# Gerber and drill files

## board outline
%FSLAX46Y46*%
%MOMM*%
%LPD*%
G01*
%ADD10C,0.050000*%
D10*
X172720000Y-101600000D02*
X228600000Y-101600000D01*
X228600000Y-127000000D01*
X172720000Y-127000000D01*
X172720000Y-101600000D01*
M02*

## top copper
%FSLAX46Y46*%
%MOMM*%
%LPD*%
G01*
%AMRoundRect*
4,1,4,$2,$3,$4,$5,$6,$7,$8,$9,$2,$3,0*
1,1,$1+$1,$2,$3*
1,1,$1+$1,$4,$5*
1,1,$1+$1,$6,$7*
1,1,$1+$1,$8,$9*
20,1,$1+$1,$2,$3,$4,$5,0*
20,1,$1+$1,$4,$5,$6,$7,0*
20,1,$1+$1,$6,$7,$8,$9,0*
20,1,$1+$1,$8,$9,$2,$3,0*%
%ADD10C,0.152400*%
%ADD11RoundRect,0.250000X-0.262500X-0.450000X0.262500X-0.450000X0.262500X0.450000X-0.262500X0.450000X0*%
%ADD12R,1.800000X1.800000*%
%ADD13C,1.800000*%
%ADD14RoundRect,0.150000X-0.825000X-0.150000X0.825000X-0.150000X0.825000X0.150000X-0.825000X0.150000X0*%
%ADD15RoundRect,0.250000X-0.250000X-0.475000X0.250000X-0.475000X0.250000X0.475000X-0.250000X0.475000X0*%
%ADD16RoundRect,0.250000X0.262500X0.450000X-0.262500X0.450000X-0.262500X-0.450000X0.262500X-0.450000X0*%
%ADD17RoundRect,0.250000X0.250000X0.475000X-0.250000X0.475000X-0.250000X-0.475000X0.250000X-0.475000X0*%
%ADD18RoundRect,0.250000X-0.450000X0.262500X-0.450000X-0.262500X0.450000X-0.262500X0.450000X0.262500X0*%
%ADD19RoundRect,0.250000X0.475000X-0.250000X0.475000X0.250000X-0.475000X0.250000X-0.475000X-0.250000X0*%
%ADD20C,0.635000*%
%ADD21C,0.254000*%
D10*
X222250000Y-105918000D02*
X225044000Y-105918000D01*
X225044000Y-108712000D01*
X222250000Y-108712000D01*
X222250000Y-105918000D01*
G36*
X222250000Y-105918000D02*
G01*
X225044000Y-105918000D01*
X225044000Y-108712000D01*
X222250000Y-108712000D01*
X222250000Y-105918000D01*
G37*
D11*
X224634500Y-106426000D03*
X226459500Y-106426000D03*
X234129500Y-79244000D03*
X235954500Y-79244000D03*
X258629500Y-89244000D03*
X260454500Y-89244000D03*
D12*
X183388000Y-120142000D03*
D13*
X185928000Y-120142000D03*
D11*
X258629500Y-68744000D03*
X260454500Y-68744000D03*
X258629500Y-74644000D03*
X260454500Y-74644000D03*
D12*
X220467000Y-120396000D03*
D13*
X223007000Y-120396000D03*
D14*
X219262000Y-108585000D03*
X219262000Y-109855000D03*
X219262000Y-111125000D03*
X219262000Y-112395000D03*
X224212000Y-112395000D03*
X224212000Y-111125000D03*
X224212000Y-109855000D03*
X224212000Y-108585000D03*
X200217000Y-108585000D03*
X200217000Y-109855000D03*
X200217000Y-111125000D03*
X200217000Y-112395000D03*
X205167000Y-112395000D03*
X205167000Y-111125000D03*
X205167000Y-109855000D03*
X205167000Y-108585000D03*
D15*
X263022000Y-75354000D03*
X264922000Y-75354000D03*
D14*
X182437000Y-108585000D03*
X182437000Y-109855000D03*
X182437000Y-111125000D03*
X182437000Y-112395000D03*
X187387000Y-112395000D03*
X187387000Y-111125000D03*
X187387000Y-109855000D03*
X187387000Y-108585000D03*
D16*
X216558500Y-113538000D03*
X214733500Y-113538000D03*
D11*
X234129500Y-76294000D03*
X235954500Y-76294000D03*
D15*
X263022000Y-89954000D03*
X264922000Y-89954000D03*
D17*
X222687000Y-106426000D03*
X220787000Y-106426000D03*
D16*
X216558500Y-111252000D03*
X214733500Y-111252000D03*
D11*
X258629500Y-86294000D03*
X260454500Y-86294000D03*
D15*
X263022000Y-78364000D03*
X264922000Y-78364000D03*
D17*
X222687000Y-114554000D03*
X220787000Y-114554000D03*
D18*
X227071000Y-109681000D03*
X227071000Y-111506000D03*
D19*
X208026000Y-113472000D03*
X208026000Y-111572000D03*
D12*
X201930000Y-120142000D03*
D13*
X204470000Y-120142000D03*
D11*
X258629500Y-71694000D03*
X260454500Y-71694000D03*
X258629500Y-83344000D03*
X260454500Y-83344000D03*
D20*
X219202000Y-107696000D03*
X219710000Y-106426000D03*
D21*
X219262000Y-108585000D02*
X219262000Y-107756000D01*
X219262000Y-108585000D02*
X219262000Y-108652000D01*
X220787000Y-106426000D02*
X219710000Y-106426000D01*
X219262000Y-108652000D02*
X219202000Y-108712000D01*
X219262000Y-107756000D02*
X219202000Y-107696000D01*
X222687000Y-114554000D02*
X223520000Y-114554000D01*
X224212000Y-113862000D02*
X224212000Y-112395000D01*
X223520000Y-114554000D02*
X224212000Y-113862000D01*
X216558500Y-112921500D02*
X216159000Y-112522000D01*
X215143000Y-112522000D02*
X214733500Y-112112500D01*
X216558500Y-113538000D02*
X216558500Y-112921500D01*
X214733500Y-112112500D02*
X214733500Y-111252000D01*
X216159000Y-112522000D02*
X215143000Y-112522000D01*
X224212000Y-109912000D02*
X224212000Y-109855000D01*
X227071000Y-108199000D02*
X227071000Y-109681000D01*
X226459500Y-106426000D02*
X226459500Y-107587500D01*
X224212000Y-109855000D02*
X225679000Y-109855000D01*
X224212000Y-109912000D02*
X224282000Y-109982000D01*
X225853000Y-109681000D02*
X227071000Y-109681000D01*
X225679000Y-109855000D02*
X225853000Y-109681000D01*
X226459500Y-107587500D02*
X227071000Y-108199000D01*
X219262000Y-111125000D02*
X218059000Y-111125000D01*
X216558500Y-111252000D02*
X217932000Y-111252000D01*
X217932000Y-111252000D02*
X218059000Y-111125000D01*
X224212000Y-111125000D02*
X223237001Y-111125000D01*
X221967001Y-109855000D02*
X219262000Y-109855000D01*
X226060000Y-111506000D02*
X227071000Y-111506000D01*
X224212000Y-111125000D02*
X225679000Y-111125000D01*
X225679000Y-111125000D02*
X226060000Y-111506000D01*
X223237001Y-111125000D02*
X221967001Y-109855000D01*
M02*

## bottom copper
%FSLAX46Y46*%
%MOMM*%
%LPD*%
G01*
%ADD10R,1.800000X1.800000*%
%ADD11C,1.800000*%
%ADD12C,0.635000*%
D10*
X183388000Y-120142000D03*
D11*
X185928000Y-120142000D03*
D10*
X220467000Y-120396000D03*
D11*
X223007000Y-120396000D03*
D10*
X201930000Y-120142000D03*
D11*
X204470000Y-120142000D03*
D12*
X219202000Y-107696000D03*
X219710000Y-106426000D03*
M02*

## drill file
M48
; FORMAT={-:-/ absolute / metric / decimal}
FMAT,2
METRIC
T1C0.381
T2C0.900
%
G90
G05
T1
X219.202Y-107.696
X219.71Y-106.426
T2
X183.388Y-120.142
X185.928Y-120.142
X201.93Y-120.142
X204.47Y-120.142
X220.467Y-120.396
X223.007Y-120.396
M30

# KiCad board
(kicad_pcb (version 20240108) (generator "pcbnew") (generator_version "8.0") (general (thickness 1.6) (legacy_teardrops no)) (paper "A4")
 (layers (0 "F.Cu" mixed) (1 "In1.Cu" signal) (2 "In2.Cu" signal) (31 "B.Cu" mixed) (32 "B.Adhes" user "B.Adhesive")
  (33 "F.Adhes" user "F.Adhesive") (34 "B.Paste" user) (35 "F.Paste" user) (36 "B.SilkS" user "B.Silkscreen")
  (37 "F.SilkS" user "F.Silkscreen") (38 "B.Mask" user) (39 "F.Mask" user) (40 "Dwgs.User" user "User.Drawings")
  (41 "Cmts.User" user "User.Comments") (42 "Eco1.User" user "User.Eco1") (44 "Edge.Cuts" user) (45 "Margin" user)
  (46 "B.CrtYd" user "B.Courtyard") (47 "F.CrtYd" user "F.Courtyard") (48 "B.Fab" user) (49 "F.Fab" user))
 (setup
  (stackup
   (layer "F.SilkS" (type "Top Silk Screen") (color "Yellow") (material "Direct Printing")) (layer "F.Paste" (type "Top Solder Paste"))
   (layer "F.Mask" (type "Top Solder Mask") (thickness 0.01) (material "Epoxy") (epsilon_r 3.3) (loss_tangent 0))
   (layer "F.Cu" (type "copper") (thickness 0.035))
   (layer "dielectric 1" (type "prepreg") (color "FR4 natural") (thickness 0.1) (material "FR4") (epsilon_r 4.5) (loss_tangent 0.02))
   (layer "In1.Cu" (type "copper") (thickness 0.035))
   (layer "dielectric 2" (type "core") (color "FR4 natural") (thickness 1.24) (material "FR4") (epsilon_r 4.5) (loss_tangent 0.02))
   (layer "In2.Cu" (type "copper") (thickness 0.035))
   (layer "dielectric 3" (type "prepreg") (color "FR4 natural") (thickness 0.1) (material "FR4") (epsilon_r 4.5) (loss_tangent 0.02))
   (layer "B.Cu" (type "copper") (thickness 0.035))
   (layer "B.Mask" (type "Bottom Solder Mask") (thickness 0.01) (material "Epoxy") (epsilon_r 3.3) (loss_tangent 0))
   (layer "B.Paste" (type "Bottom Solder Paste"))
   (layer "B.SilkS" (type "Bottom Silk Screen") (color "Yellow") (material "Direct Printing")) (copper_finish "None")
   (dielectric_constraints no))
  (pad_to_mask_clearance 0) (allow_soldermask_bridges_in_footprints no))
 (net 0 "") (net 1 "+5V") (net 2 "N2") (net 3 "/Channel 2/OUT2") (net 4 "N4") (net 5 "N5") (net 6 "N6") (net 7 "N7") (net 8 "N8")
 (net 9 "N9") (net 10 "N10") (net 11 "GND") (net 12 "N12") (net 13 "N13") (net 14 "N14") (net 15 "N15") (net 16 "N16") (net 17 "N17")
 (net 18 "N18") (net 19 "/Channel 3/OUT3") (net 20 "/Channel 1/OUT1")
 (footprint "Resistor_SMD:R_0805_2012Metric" (layer "F.Cu") (at 225.547 106.426)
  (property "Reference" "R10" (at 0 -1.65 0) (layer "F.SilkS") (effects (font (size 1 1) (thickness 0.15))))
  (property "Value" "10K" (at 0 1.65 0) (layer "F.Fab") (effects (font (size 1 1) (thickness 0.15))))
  (pad "1" smd roundrect (at -0.9125 0) (size 1.025 1.4) (layers "F.Cu" "F.Paste" "F.Mask") (roundrect_rratio 0.243902) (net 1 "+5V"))
  (pad "2" smd roundrect (at 0.9125 0) (size 1.025 1.4) (layers "F.Cu" "F.Paste" "F.Mask") (roundrect_rratio 0.243902) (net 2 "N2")))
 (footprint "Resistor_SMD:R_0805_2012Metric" (layer "F.Cu") (at 235.042 79.244)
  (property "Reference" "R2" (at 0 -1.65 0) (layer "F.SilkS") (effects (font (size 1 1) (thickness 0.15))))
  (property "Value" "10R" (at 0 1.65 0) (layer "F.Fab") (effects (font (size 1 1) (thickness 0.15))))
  (pad "1" smd roundrect (at -0.9125 0) (size 1.025 1.4) (layers "F.Cu" "F.Paste" "F.Mask") (roundrect_rratio 0.243902)
   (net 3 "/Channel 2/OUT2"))
  (pad "2" smd roundrect (at 0.9125 0) (size 1.025 1.4) (layers "F.Cu" "F.Paste" "F.Mask") (roundrect_rratio 0.243902) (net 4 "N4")))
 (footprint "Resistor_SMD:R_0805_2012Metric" (layer "F.Cu") (at 259.542 89.244)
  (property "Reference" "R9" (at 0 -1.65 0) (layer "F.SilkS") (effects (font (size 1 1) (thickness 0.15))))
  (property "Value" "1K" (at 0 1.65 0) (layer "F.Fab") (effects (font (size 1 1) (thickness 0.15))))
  (pad "1" smd roundrect (at -0.9125 0) (size 1.025 1.4) (layers "F.Cu" "F.Paste" "F.Mask") (roundrect_rratio 0.243902) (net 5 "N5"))
  (pad "2" smd roundrect (at 0.9125 0) (size 1.025 1.4) (layers "F.Cu" "F.Paste" "F.Mask") (roundrect_rratio 0.243902) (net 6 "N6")))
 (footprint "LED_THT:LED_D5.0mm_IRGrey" (layer "F.Cu") (at 183.388 120.142)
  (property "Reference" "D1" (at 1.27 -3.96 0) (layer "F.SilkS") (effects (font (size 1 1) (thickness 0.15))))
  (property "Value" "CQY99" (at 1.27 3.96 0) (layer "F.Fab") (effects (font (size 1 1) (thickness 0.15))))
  (pad "1" thru_hole rect (at 0 0) (size 1.8 1.8) (drill 0.9) (layers "*.Cu" "*.Mask") (remove_unused_layers no) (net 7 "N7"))
  (pad "2" thru_hole circle (at 2.54 0) (size 1.8 1.8) (drill 0.9) (layers "*.Cu" "*.Mask") (remove_unused_layers no) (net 1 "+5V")))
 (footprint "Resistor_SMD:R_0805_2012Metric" (layer "F.Cu") (at 259.542 68.744)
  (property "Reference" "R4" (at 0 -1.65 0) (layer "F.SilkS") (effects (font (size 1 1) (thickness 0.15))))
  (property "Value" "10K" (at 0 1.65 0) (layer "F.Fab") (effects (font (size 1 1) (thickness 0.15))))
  (pad "1" smd roundrect (at -0.9125 0) (size 1.025 1.4) (layers "F.Cu" "F.Paste" "F.Mask") (roundrect_rratio 0.243902) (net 1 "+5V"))
  (pad "2" smd roundrect (at 0.9125 0) (size 1.025 1.4) (layers "F.Cu" "F.Paste" "F.Mask") (roundrect_rratio 0.243902) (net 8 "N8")))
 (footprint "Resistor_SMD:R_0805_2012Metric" (layer "F.Cu") (at 259.542 74.644)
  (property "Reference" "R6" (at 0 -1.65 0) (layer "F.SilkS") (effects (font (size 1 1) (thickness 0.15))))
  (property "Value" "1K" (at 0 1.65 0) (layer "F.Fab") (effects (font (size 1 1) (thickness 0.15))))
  (pad "1" smd roundrect (at -0.9125 0) (size 1.025 1.4) (layers "F.Cu" "F.Paste" "F.Mask") (roundrect_rratio 0.243902) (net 8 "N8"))
  (pad "2" smd roundrect (at 0.9125 0) (size 1.025 1.4) (layers "F.Cu" "F.Paste" "F.Mask") (roundrect_rratio 0.243902) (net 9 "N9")))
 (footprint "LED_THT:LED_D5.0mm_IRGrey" (layer "F.Cu") (at 220.467 120.396)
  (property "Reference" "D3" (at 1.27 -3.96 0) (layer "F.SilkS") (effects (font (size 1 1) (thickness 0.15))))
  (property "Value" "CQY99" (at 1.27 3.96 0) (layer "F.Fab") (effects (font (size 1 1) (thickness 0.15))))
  (pad "1" thru_hole rect (at 0 0) (size 1.8 1.8) (drill 0.9) (layers "*.Cu" "*.Mask") (remove_unused_layers no) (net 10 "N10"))
  (pad "2" thru_hole circle (at 2.54 0) (size 1.8 1.8) (drill 0.9) (layers "*.Cu" "*.Mask") (remove_unused_layers no) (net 1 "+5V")))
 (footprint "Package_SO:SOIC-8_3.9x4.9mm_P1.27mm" (layer "F.Cu") (at 221.737 110.49)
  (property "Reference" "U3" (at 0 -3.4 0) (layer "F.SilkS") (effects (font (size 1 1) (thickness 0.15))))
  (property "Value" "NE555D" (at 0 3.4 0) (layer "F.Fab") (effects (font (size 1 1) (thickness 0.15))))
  (pad "1" smd roundrect (at -2.475 -1.905) (size 1.95 0.6) (layers "F.Cu" "F.Paste" "F.Mask") (roundrect_rratio 0.25) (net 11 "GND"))
  (pad "2" smd roundrect (at -2.475 -0.635) (size 1.95 0.6) (layers "F.Cu" "F.Paste" "F.Mask") (roundrect_rratio 0.25) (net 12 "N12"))
  (pad "3" smd roundrect (at -2.475 0.635) (size 1.95 0.6) (layers "F.Cu" "F.Paste" "F.Mask") (roundrect_rratio 0.25) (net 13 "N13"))
  (pad "4" smd roundrect (at -2.475 1.905) (size 1.95 0.6) (layers "F.Cu" "F.Paste" "F.Mask") (roundrect_rratio 0.25) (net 1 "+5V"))
  (pad "5" smd roundrect (at 2.475 1.905) (size 1.95 0.6) (layers "F.Cu" "F.Paste" "F.Mask") (roundrect_rratio 0.25) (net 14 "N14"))
  (pad "6" smd roundrect (at 2.475 0.635) (size 1.95 0.6) (layers "F.Cu" "F.Paste" "F.Mask") (roundrect_rratio 0.25) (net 12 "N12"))
  (pad "7" smd roundrect (at 2.475 -0.635) (size 1.95 0.6) (layers "F.Cu" "F.Paste" "F.Mask") (roundrect_rratio 0.25) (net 2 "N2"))
  (pad "8" smd roundrect (at 2.475 -1.905) (size 1.95 0.6) (layers "F.Cu" "F.Paste" "F.Mask") (roundrect_rratio 0.25) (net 1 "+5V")))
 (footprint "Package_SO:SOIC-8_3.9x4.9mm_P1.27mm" (layer "F.Cu") (at 202.692 110.49)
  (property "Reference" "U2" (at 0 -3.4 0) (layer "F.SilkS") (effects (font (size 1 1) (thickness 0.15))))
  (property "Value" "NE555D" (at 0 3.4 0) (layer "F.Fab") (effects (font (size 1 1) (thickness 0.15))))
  (pad "1" smd roundrect (at -2.475 -1.905) (size 1.95 0.6) (layers "F.Cu" "F.Paste" "F.Mask") (roundrect_rratio 0.25) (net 11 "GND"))
  (pad "2" smd roundrect (at -2.475 -0.635) (size 1.95 0.6) (layers "F.Cu" "F.Paste" "F.Mask") (roundrect_rratio 0.25) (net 6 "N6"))
  (pad "3" smd roundrect (at -2.475 0.635) (size 1.95 0.6) (layers "F.Cu" "F.Paste" "F.Mask") (roundrect_rratio 0.25) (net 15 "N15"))
  (pad "4" smd roundrect (at -2.475 1.905) (size 1.95 0.6) (layers "F.Cu" "F.Paste" "F.Mask") (roundrect_rratio 0.25) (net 1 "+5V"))
  (pad "5" smd roundrect (at 2.475 1.905) (size 1.95 0.6) (layers "F.Cu" "F.Paste" "F.Mask") (roundrect_rratio 0.25) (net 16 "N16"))
  (pad "6" smd roundrect (at 2.475 0.635) (size 1.95 0.6) (layers "F.Cu" "F.Paste" "F.Mask") (roundrect_rratio 0.25) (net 6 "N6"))
  (pad "7" smd roundrect (at 2.475 -0.635) (size 1.95 0.6) (layers "F.Cu" "F.Paste" "F.Mask") (roundrect_rratio 0.25) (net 5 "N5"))
  (pad "8" smd roundrect (at 2.475 -1.905) (size 1.95 0.6) (layers "F.Cu" "F.Paste" "F.Mask") (roundrect_rratio 0.25) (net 1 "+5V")))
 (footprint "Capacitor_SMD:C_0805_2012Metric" (layer "F.Cu") (at 263.972 75.354)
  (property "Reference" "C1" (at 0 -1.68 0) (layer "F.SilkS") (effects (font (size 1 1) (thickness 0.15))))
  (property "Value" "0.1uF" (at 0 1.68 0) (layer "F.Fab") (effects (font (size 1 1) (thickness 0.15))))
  (pad "1" smd roundrect (at -0.95 0) (size 1 1.45) (layers "F.Cu" "F.Paste" "F.Mask") (roundrect_rratio 0.25) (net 1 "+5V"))
  (pad "2" smd roundrect (at 0.95 0) (size 1 1.45) (layers "F.Cu" "F.Paste" "F.Mask") (roundrect_rratio 0.25) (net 11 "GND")))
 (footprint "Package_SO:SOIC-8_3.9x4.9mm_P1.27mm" (layer "F.Cu") (at 184.912 110.49)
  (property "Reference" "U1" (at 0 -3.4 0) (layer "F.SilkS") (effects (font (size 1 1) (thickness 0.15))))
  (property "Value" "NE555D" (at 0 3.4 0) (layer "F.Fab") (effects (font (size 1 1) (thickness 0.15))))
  (pad "1" smd roundrect (at -2.475 -1.905) (size 1.95 0.6) (layers "F.Cu" "F.Paste" "F.Mask") (roundrect_rratio 0.25) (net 11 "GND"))
  (pad "2" smd roundrect (at -2.475 -0.635) (size 1.95 0.6) (layers "F.Cu" "F.Paste" "F.Mask") (roundrect_rratio 0.25) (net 9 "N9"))
  (pad "3" smd roundrect (at -2.475 0.635) (size 1.95 0.6) (layers "F.Cu" "F.Paste" "F.Mask") (roundrect_rratio 0.25) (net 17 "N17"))
  (pad "4" smd roundrect (at -2.475 1.905) (size 1.95 0.6) (layers "F.Cu" "F.Paste" "F.Mask") (roundrect_rratio 0.25) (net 1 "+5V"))
  (pad "5" smd roundrect (at 2.475 1.905) (size 1.95 0.6) (layers "F.Cu" "F.Paste" "F.Mask") (roundrect_rratio 0.25) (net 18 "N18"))
  (pad "6" smd roundrect (at 2.475 0.635) (size 1.95 0.6) (layers "F.Cu" "F.Paste" "F.Mask") (roundrect_rratio 0.25) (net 9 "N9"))
  (pad "7" smd roundrect (at 2.475 -0.635) (size 1.95 0.6) (layers "F.Cu" "F.Paste" "F.Mask") (roundrect_rratio 0.25) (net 8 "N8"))
  (pad "8" smd roundrect (at 2.475 -1.905) (size 1.95 0.6) (layers "F.Cu" "F.Paste" "F.Mask") (roundrect_rratio 0.25) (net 1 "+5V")))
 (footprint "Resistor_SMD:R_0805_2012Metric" (layer "F.Cu") (at 215.646 113.538 180)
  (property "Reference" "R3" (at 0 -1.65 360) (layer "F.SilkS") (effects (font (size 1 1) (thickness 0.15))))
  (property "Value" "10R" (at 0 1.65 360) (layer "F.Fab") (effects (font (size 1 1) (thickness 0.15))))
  (pad "1" smd roundrect (at -0.9125 0 180) (size 1.025 1.4) (layers "F.Cu" "F.Paste" "F.Mask") (roundrect_rratio 0.243902)
   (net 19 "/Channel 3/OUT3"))
  (pad "2" smd roundrect (at 0.9125 0 180) (size 1.025 1.4) (layers "F.Cu" "F.Paste" "F.Mask") (roundrect_rratio 0.243902) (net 10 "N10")))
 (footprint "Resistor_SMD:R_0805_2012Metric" (layer "F.Cu") (at 235.042 76.294)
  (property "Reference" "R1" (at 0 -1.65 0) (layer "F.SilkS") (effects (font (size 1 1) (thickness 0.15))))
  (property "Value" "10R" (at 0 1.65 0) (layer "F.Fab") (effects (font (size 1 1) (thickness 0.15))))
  (pad "1" smd roundrect (at -0.9125 0) (size 1.025 1.4) (layers "F.Cu" "F.Paste" "F.Mask") (roundrect_rratio 0.243902)
   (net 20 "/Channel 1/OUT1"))
  (pad "2" smd roundrect (at 0.9125 0) (size 1.025 1.4) (layers "F.Cu" "F.Paste" "F.Mask") (roundrect_rratio 0.243902) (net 7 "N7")))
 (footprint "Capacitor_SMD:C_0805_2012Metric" (layer "F.Cu") (at 263.972 89.954)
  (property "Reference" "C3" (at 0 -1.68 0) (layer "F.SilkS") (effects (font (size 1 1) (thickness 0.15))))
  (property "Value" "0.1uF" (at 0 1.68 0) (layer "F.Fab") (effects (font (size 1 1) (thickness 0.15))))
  (pad "1" smd roundrect (at -0.95 0) (size 1 1.45) (layers "F.Cu" "F.Paste" "F.Mask") (roundrect_rratio 0.25) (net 1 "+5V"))
  (pad "2" smd roundrect (at 0.95 0) (size 1 1.45) (layers "F.Cu" "F.Paste" "F.Mask") (roundrect_rratio 0.25) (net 11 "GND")))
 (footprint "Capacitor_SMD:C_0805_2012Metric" (layer "F.Cu") (at 221.737 106.426 180)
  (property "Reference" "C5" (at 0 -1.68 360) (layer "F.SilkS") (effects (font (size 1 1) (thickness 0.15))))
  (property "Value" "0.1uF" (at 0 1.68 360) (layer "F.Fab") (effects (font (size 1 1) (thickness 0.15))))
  (pad "1" smd roundrect (at -0.95 0 180) (size 1 1.45) (layers "F.Cu" "F.Paste" "F.Mask") (roundrect_rratio 0.25) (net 1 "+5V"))
  (pad "2" smd roundrect (at 0.95 0 180) (size 1 1.45) (layers "F.Cu" "F.Paste" "F.Mask") (roundrect_rratio 0.25) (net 11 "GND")))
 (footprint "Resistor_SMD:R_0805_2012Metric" (layer "F.Cu") (at 215.646 111.252 180)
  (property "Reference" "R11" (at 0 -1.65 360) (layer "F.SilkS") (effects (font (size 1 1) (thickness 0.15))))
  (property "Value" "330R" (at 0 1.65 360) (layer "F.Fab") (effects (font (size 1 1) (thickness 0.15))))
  (pad "1" smd roundrect (at -0.9125 0 180) (size 1.025 1.4) (layers "F.Cu" "F.Paste" "F.Mask") (roundrect_rratio 0.243902) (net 13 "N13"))
  (pad "2" smd roundrect (at 0.9125 0 180) (size 1.025 1.4) (layers "F.Cu" "F.Paste" "F.Mask") (roundrect_rratio 0.243902)
   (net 19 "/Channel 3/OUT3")))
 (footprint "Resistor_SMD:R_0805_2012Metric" (layer "F.Cu") (at 259.542 86.294)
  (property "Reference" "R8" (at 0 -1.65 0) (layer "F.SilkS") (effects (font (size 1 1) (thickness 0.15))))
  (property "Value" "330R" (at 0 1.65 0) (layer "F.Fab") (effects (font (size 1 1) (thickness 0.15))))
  (pad "1" smd roundrect (at -0.9125 0) (size 1.025 1.4) (layers "F.Cu" "F.Paste" "F.Mask") (roundrect_rratio 0.243902) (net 15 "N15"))
  (pad "2" smd roundrect (at 0.9125 0) (size 1.025 1.4) (layers "F.Cu" "F.Paste" "F.Mask") (roundrect_rratio 0.243902)
   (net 3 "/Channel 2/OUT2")))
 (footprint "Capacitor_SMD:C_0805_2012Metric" (layer "F.Cu") (at 263.972 78.364)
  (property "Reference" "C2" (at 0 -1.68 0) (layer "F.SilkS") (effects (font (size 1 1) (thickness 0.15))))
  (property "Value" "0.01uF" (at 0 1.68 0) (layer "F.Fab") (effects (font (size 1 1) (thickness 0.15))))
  (pad "1" smd roundrect (at -0.95 0) (size 1 1.45) (layers "F.Cu" "F.Paste" "F.Mask") (roundrect_rratio 0.25) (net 18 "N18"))
  (pad "2" smd roundrect (at 0.95 0) (size 1 1.45) (layers "F.Cu" "F.Paste" "F.Mask") (roundrect_rratio 0.25) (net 11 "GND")))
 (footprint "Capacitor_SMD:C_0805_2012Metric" (layer "F.Cu") (at 221.737 114.554 180)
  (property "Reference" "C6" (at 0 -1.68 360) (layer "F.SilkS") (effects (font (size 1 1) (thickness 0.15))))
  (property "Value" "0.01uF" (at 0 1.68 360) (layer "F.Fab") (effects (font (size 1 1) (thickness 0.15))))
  (pad "1" smd roundrect (at -0.95 0 180) (size 1 1.45) (layers "F.Cu" "F.Paste" "F.Mask") (roundrect_rratio 0.25) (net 14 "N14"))
  (pad "2" smd roundrect (at 0.95 0 180) (size 1 1.45) (layers "F.Cu" "F.Paste" "F.Mask") (roundrect_rratio 0.25) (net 11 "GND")))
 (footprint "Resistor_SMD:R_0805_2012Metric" (layer "F.Cu") (at 227.071 110.5935 -90)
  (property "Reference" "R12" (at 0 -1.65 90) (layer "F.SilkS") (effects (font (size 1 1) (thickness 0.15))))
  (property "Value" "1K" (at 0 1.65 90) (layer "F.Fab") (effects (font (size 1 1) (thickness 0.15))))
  (pad "1" smd roundrect (at -0.9125 0 270) (size 1.025 1.4) (layers "F.Cu" "F.Paste" "F.Mask") (roundrect_rratio 0.243902) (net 2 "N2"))
  (pad "2" smd roundrect (at 0.9125 0 270) (size 1.025 1.4) (layers "F.Cu" "F.Paste" "F.Mask") (roundrect_rratio 0.243902) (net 12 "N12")))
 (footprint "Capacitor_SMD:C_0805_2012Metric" (layer "F.Cu") (at 208.026 112.522 90)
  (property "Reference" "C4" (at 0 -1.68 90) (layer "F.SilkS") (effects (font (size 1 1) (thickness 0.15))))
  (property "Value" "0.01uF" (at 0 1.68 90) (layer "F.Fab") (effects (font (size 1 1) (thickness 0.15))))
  (pad "1" smd roundrect (at -0.95 0 90) (size 1 1.45) (layers "F.Cu" "F.Paste" "F.Mask") (roundrect_rratio 0.25) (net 16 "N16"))
  (pad "2" smd roundrect (at 0.95 0 90) (size 1 1.45) (layers "F.Cu" "F.Paste" "F.Mask") (roundrect_rratio 0.25) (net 11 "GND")))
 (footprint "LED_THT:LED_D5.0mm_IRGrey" (layer "F.Cu") (at 201.93 120.142)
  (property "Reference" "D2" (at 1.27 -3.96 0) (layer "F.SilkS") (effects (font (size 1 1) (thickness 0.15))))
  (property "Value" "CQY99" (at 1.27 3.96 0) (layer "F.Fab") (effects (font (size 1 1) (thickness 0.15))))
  (pad "1" thru_hole rect (at 0 0) (size 1.8 1.8) (drill 0.9) (layers "*.Cu" "*.Mask") (remove_unused_layers no) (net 4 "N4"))
  (pad "2" thru_hole circle (at 2.54 0) (size 1.8 1.8) (drill 0.9) (layers "*.Cu" "*.Mask") (remove_unused_layers no) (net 1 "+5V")))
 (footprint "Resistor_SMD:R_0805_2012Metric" (layer "F.Cu") (at 259.542 71.694)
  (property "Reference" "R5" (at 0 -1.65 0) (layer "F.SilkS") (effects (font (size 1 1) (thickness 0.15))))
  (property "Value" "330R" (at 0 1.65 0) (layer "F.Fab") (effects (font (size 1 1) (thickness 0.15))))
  (pad "1" smd roundrect (at -0.9125 0) (size 1.025 1.4) (layers "F.Cu" "F.Paste" "F.Mask") (roundrect_rratio 0.243902) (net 17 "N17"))
  (pad "2" smd roundrect (at 0.9125 0) (size 1.025 1.4) (layers "F.Cu" "F.Paste" "F.Mask") (roundrect_rratio 0.243902)
   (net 20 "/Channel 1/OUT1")))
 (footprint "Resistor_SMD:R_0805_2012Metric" (layer "F.Cu") (at 259.542 83.344)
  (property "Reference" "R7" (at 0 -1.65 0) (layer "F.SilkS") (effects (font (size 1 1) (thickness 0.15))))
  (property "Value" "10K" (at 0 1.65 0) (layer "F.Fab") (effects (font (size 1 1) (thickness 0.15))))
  (pad "1" smd roundrect (at -0.9125 0) (size 1.025 1.4) (layers "F.Cu" "F.Paste" "F.Mask") (roundrect_rratio 0.243902) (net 1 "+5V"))
  (pad "2" smd roundrect (at 0.9125 0) (size 1.025 1.4) (layers "F.Cu" "F.Paste" "F.Mask") (roundrect_rratio 0.243902) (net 5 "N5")))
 (gr_rect (start 222.25 105.918) (end 225.044 108.712) (stroke (width 0.1524) (type solid)) (fill solid) (layer "F.Cu") (net 1))
 (gr_rect (start 172.72 101.6) (end 228.6 127) (stroke (width 0.05) (type default)) (fill none) (layer "Edge.Cuts"))
 (segment (start 219.262 108.585) (end 219.262 107.756) (width 0.254) (layer "F.Cu") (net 11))
 (segment (start 219.262 108.585) (end 219.262 108.652) (width 0.254) (layer "F.Cu") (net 11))
 (segment (start 220.787 106.426) (end 219.71 106.426) (width 0.254) (layer "F.Cu") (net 11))
 (segment (start 219.262 108.652) (end 219.202 108.712) (width 0.254) (layer "F.Cu") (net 11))
 (segment (start 219.262 107.756) (end 219.202 107.696) (width 0.254) (layer "F.Cu") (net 11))
 (via (at 219.202 107.696) (size 0.635) (drill 0.381) (layers "F.Cu" "B.Cu") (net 11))
 (via (at 219.71 106.426) (size 0.635) (drill 0.381) (layers "F.Cu" "B.Cu")
  (teardrops (best_length_ratio 0.5) (max_length 1) (best_width_ratio 1) (max_width 2) (curve_points 0) (filter_ratio 0.9) (enabled no)
   (allow_two_segments no) (prefer_zone_connections yes))
  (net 11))
 (segment (start 222.687 114.554) (end 223.52 114.554) (width 0.254) (layer "F.Cu") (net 14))
 (segment (start 224.212 113.862) (end 224.212 112.395) (width 0.254) (layer "F.Cu") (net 14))
 (segment (start 223.52 114.554) (end 224.212 113.862) (width 0.254) (layer "F.Cu") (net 14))
 (segment (start 216.5585 112.9215) (end 216.159 112.522) (width 0.254) (layer "F.Cu") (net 19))
 (segment (start 215.143 112.522) (end 214.7335 112.1125) (width 0.254) (layer "F.Cu") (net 19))
 (segment (start 216.5585 113.538) (end 216.5585 112.9215) (width 0.254) (layer "F.Cu") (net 19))
 (segment (start 214.7335 112.1125) (end 214.7335 111.252) (width 0.254) (layer "F.Cu") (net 19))
 (segment (start 216.159 112.522) (end 215.143 112.522) (width 0.254) (layer "F.Cu") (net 19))
 (segment (start 224.212 109.912) (end 224.212 109.855) (width 0.254) (layer "F.Cu") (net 2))
 (segment (start 227.071 108.199) (end 227.071 109.681) (width 0.254) (layer "F.Cu") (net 2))
 (segment (start 226.4595 106.426) (end 226.4595 107.5875) (width 0.254) (layer "F.Cu") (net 2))
 (segment (start 224.212 109.855) (end 225.679 109.855) (width 0.254) (layer "F.Cu") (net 2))
 (segment (start 224.212 109.912) (end 224.282 109.982) (width 0.254) (layer "F.Cu") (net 2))
 (segment (start 225.853 109.681) (end 227.071 109.681) (width 0.254) (layer "F.Cu") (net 2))
 (segment (start 225.679 109.855) (end 225.853 109.681) (width 0.254) (layer "F.Cu") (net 2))
 (segment (start 226.4595 107.5875) (end 227.071 108.199) (width 0.254) (layer "F.Cu") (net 2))
 (segment (start 219.262 111.125) (end 218.059 111.125) (width 0.254) (layer "F.Cu") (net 13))
 (segment (start 216.5585 111.252) (end 217.932 111.252) (width 0.254) (layer "F.Cu") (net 13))
 (segment (start 217.932 111.252) (end 218.059 111.125) (width 0.254) (layer "F.Cu") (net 13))
 (segment (start 224.212 111.125) (end 223.237001 111.125) (width 0.254) (layer "F.Cu") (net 12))
 (segment (start 221.967001 109.855) (end 219.262 109.855) (width 0.254) (layer "F.Cu") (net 12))
 (segment (start 226.06 111.506) (end 227.071 111.506) (width 0.254) (layer "F.Cu") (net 12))
 (segment (start 224.212 111.125) (end 225.679 111.125) (width 0.254) (layer "F.Cu") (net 12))
 (segment (start 225.679 111.125) (end 226.06 111.506) (width 0.254) (layer "F.Cu") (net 12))
 (segment (start 223.237001 111.125) (end 221.967001 109.855) (width 0.254) (layer "F.Cu") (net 12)))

